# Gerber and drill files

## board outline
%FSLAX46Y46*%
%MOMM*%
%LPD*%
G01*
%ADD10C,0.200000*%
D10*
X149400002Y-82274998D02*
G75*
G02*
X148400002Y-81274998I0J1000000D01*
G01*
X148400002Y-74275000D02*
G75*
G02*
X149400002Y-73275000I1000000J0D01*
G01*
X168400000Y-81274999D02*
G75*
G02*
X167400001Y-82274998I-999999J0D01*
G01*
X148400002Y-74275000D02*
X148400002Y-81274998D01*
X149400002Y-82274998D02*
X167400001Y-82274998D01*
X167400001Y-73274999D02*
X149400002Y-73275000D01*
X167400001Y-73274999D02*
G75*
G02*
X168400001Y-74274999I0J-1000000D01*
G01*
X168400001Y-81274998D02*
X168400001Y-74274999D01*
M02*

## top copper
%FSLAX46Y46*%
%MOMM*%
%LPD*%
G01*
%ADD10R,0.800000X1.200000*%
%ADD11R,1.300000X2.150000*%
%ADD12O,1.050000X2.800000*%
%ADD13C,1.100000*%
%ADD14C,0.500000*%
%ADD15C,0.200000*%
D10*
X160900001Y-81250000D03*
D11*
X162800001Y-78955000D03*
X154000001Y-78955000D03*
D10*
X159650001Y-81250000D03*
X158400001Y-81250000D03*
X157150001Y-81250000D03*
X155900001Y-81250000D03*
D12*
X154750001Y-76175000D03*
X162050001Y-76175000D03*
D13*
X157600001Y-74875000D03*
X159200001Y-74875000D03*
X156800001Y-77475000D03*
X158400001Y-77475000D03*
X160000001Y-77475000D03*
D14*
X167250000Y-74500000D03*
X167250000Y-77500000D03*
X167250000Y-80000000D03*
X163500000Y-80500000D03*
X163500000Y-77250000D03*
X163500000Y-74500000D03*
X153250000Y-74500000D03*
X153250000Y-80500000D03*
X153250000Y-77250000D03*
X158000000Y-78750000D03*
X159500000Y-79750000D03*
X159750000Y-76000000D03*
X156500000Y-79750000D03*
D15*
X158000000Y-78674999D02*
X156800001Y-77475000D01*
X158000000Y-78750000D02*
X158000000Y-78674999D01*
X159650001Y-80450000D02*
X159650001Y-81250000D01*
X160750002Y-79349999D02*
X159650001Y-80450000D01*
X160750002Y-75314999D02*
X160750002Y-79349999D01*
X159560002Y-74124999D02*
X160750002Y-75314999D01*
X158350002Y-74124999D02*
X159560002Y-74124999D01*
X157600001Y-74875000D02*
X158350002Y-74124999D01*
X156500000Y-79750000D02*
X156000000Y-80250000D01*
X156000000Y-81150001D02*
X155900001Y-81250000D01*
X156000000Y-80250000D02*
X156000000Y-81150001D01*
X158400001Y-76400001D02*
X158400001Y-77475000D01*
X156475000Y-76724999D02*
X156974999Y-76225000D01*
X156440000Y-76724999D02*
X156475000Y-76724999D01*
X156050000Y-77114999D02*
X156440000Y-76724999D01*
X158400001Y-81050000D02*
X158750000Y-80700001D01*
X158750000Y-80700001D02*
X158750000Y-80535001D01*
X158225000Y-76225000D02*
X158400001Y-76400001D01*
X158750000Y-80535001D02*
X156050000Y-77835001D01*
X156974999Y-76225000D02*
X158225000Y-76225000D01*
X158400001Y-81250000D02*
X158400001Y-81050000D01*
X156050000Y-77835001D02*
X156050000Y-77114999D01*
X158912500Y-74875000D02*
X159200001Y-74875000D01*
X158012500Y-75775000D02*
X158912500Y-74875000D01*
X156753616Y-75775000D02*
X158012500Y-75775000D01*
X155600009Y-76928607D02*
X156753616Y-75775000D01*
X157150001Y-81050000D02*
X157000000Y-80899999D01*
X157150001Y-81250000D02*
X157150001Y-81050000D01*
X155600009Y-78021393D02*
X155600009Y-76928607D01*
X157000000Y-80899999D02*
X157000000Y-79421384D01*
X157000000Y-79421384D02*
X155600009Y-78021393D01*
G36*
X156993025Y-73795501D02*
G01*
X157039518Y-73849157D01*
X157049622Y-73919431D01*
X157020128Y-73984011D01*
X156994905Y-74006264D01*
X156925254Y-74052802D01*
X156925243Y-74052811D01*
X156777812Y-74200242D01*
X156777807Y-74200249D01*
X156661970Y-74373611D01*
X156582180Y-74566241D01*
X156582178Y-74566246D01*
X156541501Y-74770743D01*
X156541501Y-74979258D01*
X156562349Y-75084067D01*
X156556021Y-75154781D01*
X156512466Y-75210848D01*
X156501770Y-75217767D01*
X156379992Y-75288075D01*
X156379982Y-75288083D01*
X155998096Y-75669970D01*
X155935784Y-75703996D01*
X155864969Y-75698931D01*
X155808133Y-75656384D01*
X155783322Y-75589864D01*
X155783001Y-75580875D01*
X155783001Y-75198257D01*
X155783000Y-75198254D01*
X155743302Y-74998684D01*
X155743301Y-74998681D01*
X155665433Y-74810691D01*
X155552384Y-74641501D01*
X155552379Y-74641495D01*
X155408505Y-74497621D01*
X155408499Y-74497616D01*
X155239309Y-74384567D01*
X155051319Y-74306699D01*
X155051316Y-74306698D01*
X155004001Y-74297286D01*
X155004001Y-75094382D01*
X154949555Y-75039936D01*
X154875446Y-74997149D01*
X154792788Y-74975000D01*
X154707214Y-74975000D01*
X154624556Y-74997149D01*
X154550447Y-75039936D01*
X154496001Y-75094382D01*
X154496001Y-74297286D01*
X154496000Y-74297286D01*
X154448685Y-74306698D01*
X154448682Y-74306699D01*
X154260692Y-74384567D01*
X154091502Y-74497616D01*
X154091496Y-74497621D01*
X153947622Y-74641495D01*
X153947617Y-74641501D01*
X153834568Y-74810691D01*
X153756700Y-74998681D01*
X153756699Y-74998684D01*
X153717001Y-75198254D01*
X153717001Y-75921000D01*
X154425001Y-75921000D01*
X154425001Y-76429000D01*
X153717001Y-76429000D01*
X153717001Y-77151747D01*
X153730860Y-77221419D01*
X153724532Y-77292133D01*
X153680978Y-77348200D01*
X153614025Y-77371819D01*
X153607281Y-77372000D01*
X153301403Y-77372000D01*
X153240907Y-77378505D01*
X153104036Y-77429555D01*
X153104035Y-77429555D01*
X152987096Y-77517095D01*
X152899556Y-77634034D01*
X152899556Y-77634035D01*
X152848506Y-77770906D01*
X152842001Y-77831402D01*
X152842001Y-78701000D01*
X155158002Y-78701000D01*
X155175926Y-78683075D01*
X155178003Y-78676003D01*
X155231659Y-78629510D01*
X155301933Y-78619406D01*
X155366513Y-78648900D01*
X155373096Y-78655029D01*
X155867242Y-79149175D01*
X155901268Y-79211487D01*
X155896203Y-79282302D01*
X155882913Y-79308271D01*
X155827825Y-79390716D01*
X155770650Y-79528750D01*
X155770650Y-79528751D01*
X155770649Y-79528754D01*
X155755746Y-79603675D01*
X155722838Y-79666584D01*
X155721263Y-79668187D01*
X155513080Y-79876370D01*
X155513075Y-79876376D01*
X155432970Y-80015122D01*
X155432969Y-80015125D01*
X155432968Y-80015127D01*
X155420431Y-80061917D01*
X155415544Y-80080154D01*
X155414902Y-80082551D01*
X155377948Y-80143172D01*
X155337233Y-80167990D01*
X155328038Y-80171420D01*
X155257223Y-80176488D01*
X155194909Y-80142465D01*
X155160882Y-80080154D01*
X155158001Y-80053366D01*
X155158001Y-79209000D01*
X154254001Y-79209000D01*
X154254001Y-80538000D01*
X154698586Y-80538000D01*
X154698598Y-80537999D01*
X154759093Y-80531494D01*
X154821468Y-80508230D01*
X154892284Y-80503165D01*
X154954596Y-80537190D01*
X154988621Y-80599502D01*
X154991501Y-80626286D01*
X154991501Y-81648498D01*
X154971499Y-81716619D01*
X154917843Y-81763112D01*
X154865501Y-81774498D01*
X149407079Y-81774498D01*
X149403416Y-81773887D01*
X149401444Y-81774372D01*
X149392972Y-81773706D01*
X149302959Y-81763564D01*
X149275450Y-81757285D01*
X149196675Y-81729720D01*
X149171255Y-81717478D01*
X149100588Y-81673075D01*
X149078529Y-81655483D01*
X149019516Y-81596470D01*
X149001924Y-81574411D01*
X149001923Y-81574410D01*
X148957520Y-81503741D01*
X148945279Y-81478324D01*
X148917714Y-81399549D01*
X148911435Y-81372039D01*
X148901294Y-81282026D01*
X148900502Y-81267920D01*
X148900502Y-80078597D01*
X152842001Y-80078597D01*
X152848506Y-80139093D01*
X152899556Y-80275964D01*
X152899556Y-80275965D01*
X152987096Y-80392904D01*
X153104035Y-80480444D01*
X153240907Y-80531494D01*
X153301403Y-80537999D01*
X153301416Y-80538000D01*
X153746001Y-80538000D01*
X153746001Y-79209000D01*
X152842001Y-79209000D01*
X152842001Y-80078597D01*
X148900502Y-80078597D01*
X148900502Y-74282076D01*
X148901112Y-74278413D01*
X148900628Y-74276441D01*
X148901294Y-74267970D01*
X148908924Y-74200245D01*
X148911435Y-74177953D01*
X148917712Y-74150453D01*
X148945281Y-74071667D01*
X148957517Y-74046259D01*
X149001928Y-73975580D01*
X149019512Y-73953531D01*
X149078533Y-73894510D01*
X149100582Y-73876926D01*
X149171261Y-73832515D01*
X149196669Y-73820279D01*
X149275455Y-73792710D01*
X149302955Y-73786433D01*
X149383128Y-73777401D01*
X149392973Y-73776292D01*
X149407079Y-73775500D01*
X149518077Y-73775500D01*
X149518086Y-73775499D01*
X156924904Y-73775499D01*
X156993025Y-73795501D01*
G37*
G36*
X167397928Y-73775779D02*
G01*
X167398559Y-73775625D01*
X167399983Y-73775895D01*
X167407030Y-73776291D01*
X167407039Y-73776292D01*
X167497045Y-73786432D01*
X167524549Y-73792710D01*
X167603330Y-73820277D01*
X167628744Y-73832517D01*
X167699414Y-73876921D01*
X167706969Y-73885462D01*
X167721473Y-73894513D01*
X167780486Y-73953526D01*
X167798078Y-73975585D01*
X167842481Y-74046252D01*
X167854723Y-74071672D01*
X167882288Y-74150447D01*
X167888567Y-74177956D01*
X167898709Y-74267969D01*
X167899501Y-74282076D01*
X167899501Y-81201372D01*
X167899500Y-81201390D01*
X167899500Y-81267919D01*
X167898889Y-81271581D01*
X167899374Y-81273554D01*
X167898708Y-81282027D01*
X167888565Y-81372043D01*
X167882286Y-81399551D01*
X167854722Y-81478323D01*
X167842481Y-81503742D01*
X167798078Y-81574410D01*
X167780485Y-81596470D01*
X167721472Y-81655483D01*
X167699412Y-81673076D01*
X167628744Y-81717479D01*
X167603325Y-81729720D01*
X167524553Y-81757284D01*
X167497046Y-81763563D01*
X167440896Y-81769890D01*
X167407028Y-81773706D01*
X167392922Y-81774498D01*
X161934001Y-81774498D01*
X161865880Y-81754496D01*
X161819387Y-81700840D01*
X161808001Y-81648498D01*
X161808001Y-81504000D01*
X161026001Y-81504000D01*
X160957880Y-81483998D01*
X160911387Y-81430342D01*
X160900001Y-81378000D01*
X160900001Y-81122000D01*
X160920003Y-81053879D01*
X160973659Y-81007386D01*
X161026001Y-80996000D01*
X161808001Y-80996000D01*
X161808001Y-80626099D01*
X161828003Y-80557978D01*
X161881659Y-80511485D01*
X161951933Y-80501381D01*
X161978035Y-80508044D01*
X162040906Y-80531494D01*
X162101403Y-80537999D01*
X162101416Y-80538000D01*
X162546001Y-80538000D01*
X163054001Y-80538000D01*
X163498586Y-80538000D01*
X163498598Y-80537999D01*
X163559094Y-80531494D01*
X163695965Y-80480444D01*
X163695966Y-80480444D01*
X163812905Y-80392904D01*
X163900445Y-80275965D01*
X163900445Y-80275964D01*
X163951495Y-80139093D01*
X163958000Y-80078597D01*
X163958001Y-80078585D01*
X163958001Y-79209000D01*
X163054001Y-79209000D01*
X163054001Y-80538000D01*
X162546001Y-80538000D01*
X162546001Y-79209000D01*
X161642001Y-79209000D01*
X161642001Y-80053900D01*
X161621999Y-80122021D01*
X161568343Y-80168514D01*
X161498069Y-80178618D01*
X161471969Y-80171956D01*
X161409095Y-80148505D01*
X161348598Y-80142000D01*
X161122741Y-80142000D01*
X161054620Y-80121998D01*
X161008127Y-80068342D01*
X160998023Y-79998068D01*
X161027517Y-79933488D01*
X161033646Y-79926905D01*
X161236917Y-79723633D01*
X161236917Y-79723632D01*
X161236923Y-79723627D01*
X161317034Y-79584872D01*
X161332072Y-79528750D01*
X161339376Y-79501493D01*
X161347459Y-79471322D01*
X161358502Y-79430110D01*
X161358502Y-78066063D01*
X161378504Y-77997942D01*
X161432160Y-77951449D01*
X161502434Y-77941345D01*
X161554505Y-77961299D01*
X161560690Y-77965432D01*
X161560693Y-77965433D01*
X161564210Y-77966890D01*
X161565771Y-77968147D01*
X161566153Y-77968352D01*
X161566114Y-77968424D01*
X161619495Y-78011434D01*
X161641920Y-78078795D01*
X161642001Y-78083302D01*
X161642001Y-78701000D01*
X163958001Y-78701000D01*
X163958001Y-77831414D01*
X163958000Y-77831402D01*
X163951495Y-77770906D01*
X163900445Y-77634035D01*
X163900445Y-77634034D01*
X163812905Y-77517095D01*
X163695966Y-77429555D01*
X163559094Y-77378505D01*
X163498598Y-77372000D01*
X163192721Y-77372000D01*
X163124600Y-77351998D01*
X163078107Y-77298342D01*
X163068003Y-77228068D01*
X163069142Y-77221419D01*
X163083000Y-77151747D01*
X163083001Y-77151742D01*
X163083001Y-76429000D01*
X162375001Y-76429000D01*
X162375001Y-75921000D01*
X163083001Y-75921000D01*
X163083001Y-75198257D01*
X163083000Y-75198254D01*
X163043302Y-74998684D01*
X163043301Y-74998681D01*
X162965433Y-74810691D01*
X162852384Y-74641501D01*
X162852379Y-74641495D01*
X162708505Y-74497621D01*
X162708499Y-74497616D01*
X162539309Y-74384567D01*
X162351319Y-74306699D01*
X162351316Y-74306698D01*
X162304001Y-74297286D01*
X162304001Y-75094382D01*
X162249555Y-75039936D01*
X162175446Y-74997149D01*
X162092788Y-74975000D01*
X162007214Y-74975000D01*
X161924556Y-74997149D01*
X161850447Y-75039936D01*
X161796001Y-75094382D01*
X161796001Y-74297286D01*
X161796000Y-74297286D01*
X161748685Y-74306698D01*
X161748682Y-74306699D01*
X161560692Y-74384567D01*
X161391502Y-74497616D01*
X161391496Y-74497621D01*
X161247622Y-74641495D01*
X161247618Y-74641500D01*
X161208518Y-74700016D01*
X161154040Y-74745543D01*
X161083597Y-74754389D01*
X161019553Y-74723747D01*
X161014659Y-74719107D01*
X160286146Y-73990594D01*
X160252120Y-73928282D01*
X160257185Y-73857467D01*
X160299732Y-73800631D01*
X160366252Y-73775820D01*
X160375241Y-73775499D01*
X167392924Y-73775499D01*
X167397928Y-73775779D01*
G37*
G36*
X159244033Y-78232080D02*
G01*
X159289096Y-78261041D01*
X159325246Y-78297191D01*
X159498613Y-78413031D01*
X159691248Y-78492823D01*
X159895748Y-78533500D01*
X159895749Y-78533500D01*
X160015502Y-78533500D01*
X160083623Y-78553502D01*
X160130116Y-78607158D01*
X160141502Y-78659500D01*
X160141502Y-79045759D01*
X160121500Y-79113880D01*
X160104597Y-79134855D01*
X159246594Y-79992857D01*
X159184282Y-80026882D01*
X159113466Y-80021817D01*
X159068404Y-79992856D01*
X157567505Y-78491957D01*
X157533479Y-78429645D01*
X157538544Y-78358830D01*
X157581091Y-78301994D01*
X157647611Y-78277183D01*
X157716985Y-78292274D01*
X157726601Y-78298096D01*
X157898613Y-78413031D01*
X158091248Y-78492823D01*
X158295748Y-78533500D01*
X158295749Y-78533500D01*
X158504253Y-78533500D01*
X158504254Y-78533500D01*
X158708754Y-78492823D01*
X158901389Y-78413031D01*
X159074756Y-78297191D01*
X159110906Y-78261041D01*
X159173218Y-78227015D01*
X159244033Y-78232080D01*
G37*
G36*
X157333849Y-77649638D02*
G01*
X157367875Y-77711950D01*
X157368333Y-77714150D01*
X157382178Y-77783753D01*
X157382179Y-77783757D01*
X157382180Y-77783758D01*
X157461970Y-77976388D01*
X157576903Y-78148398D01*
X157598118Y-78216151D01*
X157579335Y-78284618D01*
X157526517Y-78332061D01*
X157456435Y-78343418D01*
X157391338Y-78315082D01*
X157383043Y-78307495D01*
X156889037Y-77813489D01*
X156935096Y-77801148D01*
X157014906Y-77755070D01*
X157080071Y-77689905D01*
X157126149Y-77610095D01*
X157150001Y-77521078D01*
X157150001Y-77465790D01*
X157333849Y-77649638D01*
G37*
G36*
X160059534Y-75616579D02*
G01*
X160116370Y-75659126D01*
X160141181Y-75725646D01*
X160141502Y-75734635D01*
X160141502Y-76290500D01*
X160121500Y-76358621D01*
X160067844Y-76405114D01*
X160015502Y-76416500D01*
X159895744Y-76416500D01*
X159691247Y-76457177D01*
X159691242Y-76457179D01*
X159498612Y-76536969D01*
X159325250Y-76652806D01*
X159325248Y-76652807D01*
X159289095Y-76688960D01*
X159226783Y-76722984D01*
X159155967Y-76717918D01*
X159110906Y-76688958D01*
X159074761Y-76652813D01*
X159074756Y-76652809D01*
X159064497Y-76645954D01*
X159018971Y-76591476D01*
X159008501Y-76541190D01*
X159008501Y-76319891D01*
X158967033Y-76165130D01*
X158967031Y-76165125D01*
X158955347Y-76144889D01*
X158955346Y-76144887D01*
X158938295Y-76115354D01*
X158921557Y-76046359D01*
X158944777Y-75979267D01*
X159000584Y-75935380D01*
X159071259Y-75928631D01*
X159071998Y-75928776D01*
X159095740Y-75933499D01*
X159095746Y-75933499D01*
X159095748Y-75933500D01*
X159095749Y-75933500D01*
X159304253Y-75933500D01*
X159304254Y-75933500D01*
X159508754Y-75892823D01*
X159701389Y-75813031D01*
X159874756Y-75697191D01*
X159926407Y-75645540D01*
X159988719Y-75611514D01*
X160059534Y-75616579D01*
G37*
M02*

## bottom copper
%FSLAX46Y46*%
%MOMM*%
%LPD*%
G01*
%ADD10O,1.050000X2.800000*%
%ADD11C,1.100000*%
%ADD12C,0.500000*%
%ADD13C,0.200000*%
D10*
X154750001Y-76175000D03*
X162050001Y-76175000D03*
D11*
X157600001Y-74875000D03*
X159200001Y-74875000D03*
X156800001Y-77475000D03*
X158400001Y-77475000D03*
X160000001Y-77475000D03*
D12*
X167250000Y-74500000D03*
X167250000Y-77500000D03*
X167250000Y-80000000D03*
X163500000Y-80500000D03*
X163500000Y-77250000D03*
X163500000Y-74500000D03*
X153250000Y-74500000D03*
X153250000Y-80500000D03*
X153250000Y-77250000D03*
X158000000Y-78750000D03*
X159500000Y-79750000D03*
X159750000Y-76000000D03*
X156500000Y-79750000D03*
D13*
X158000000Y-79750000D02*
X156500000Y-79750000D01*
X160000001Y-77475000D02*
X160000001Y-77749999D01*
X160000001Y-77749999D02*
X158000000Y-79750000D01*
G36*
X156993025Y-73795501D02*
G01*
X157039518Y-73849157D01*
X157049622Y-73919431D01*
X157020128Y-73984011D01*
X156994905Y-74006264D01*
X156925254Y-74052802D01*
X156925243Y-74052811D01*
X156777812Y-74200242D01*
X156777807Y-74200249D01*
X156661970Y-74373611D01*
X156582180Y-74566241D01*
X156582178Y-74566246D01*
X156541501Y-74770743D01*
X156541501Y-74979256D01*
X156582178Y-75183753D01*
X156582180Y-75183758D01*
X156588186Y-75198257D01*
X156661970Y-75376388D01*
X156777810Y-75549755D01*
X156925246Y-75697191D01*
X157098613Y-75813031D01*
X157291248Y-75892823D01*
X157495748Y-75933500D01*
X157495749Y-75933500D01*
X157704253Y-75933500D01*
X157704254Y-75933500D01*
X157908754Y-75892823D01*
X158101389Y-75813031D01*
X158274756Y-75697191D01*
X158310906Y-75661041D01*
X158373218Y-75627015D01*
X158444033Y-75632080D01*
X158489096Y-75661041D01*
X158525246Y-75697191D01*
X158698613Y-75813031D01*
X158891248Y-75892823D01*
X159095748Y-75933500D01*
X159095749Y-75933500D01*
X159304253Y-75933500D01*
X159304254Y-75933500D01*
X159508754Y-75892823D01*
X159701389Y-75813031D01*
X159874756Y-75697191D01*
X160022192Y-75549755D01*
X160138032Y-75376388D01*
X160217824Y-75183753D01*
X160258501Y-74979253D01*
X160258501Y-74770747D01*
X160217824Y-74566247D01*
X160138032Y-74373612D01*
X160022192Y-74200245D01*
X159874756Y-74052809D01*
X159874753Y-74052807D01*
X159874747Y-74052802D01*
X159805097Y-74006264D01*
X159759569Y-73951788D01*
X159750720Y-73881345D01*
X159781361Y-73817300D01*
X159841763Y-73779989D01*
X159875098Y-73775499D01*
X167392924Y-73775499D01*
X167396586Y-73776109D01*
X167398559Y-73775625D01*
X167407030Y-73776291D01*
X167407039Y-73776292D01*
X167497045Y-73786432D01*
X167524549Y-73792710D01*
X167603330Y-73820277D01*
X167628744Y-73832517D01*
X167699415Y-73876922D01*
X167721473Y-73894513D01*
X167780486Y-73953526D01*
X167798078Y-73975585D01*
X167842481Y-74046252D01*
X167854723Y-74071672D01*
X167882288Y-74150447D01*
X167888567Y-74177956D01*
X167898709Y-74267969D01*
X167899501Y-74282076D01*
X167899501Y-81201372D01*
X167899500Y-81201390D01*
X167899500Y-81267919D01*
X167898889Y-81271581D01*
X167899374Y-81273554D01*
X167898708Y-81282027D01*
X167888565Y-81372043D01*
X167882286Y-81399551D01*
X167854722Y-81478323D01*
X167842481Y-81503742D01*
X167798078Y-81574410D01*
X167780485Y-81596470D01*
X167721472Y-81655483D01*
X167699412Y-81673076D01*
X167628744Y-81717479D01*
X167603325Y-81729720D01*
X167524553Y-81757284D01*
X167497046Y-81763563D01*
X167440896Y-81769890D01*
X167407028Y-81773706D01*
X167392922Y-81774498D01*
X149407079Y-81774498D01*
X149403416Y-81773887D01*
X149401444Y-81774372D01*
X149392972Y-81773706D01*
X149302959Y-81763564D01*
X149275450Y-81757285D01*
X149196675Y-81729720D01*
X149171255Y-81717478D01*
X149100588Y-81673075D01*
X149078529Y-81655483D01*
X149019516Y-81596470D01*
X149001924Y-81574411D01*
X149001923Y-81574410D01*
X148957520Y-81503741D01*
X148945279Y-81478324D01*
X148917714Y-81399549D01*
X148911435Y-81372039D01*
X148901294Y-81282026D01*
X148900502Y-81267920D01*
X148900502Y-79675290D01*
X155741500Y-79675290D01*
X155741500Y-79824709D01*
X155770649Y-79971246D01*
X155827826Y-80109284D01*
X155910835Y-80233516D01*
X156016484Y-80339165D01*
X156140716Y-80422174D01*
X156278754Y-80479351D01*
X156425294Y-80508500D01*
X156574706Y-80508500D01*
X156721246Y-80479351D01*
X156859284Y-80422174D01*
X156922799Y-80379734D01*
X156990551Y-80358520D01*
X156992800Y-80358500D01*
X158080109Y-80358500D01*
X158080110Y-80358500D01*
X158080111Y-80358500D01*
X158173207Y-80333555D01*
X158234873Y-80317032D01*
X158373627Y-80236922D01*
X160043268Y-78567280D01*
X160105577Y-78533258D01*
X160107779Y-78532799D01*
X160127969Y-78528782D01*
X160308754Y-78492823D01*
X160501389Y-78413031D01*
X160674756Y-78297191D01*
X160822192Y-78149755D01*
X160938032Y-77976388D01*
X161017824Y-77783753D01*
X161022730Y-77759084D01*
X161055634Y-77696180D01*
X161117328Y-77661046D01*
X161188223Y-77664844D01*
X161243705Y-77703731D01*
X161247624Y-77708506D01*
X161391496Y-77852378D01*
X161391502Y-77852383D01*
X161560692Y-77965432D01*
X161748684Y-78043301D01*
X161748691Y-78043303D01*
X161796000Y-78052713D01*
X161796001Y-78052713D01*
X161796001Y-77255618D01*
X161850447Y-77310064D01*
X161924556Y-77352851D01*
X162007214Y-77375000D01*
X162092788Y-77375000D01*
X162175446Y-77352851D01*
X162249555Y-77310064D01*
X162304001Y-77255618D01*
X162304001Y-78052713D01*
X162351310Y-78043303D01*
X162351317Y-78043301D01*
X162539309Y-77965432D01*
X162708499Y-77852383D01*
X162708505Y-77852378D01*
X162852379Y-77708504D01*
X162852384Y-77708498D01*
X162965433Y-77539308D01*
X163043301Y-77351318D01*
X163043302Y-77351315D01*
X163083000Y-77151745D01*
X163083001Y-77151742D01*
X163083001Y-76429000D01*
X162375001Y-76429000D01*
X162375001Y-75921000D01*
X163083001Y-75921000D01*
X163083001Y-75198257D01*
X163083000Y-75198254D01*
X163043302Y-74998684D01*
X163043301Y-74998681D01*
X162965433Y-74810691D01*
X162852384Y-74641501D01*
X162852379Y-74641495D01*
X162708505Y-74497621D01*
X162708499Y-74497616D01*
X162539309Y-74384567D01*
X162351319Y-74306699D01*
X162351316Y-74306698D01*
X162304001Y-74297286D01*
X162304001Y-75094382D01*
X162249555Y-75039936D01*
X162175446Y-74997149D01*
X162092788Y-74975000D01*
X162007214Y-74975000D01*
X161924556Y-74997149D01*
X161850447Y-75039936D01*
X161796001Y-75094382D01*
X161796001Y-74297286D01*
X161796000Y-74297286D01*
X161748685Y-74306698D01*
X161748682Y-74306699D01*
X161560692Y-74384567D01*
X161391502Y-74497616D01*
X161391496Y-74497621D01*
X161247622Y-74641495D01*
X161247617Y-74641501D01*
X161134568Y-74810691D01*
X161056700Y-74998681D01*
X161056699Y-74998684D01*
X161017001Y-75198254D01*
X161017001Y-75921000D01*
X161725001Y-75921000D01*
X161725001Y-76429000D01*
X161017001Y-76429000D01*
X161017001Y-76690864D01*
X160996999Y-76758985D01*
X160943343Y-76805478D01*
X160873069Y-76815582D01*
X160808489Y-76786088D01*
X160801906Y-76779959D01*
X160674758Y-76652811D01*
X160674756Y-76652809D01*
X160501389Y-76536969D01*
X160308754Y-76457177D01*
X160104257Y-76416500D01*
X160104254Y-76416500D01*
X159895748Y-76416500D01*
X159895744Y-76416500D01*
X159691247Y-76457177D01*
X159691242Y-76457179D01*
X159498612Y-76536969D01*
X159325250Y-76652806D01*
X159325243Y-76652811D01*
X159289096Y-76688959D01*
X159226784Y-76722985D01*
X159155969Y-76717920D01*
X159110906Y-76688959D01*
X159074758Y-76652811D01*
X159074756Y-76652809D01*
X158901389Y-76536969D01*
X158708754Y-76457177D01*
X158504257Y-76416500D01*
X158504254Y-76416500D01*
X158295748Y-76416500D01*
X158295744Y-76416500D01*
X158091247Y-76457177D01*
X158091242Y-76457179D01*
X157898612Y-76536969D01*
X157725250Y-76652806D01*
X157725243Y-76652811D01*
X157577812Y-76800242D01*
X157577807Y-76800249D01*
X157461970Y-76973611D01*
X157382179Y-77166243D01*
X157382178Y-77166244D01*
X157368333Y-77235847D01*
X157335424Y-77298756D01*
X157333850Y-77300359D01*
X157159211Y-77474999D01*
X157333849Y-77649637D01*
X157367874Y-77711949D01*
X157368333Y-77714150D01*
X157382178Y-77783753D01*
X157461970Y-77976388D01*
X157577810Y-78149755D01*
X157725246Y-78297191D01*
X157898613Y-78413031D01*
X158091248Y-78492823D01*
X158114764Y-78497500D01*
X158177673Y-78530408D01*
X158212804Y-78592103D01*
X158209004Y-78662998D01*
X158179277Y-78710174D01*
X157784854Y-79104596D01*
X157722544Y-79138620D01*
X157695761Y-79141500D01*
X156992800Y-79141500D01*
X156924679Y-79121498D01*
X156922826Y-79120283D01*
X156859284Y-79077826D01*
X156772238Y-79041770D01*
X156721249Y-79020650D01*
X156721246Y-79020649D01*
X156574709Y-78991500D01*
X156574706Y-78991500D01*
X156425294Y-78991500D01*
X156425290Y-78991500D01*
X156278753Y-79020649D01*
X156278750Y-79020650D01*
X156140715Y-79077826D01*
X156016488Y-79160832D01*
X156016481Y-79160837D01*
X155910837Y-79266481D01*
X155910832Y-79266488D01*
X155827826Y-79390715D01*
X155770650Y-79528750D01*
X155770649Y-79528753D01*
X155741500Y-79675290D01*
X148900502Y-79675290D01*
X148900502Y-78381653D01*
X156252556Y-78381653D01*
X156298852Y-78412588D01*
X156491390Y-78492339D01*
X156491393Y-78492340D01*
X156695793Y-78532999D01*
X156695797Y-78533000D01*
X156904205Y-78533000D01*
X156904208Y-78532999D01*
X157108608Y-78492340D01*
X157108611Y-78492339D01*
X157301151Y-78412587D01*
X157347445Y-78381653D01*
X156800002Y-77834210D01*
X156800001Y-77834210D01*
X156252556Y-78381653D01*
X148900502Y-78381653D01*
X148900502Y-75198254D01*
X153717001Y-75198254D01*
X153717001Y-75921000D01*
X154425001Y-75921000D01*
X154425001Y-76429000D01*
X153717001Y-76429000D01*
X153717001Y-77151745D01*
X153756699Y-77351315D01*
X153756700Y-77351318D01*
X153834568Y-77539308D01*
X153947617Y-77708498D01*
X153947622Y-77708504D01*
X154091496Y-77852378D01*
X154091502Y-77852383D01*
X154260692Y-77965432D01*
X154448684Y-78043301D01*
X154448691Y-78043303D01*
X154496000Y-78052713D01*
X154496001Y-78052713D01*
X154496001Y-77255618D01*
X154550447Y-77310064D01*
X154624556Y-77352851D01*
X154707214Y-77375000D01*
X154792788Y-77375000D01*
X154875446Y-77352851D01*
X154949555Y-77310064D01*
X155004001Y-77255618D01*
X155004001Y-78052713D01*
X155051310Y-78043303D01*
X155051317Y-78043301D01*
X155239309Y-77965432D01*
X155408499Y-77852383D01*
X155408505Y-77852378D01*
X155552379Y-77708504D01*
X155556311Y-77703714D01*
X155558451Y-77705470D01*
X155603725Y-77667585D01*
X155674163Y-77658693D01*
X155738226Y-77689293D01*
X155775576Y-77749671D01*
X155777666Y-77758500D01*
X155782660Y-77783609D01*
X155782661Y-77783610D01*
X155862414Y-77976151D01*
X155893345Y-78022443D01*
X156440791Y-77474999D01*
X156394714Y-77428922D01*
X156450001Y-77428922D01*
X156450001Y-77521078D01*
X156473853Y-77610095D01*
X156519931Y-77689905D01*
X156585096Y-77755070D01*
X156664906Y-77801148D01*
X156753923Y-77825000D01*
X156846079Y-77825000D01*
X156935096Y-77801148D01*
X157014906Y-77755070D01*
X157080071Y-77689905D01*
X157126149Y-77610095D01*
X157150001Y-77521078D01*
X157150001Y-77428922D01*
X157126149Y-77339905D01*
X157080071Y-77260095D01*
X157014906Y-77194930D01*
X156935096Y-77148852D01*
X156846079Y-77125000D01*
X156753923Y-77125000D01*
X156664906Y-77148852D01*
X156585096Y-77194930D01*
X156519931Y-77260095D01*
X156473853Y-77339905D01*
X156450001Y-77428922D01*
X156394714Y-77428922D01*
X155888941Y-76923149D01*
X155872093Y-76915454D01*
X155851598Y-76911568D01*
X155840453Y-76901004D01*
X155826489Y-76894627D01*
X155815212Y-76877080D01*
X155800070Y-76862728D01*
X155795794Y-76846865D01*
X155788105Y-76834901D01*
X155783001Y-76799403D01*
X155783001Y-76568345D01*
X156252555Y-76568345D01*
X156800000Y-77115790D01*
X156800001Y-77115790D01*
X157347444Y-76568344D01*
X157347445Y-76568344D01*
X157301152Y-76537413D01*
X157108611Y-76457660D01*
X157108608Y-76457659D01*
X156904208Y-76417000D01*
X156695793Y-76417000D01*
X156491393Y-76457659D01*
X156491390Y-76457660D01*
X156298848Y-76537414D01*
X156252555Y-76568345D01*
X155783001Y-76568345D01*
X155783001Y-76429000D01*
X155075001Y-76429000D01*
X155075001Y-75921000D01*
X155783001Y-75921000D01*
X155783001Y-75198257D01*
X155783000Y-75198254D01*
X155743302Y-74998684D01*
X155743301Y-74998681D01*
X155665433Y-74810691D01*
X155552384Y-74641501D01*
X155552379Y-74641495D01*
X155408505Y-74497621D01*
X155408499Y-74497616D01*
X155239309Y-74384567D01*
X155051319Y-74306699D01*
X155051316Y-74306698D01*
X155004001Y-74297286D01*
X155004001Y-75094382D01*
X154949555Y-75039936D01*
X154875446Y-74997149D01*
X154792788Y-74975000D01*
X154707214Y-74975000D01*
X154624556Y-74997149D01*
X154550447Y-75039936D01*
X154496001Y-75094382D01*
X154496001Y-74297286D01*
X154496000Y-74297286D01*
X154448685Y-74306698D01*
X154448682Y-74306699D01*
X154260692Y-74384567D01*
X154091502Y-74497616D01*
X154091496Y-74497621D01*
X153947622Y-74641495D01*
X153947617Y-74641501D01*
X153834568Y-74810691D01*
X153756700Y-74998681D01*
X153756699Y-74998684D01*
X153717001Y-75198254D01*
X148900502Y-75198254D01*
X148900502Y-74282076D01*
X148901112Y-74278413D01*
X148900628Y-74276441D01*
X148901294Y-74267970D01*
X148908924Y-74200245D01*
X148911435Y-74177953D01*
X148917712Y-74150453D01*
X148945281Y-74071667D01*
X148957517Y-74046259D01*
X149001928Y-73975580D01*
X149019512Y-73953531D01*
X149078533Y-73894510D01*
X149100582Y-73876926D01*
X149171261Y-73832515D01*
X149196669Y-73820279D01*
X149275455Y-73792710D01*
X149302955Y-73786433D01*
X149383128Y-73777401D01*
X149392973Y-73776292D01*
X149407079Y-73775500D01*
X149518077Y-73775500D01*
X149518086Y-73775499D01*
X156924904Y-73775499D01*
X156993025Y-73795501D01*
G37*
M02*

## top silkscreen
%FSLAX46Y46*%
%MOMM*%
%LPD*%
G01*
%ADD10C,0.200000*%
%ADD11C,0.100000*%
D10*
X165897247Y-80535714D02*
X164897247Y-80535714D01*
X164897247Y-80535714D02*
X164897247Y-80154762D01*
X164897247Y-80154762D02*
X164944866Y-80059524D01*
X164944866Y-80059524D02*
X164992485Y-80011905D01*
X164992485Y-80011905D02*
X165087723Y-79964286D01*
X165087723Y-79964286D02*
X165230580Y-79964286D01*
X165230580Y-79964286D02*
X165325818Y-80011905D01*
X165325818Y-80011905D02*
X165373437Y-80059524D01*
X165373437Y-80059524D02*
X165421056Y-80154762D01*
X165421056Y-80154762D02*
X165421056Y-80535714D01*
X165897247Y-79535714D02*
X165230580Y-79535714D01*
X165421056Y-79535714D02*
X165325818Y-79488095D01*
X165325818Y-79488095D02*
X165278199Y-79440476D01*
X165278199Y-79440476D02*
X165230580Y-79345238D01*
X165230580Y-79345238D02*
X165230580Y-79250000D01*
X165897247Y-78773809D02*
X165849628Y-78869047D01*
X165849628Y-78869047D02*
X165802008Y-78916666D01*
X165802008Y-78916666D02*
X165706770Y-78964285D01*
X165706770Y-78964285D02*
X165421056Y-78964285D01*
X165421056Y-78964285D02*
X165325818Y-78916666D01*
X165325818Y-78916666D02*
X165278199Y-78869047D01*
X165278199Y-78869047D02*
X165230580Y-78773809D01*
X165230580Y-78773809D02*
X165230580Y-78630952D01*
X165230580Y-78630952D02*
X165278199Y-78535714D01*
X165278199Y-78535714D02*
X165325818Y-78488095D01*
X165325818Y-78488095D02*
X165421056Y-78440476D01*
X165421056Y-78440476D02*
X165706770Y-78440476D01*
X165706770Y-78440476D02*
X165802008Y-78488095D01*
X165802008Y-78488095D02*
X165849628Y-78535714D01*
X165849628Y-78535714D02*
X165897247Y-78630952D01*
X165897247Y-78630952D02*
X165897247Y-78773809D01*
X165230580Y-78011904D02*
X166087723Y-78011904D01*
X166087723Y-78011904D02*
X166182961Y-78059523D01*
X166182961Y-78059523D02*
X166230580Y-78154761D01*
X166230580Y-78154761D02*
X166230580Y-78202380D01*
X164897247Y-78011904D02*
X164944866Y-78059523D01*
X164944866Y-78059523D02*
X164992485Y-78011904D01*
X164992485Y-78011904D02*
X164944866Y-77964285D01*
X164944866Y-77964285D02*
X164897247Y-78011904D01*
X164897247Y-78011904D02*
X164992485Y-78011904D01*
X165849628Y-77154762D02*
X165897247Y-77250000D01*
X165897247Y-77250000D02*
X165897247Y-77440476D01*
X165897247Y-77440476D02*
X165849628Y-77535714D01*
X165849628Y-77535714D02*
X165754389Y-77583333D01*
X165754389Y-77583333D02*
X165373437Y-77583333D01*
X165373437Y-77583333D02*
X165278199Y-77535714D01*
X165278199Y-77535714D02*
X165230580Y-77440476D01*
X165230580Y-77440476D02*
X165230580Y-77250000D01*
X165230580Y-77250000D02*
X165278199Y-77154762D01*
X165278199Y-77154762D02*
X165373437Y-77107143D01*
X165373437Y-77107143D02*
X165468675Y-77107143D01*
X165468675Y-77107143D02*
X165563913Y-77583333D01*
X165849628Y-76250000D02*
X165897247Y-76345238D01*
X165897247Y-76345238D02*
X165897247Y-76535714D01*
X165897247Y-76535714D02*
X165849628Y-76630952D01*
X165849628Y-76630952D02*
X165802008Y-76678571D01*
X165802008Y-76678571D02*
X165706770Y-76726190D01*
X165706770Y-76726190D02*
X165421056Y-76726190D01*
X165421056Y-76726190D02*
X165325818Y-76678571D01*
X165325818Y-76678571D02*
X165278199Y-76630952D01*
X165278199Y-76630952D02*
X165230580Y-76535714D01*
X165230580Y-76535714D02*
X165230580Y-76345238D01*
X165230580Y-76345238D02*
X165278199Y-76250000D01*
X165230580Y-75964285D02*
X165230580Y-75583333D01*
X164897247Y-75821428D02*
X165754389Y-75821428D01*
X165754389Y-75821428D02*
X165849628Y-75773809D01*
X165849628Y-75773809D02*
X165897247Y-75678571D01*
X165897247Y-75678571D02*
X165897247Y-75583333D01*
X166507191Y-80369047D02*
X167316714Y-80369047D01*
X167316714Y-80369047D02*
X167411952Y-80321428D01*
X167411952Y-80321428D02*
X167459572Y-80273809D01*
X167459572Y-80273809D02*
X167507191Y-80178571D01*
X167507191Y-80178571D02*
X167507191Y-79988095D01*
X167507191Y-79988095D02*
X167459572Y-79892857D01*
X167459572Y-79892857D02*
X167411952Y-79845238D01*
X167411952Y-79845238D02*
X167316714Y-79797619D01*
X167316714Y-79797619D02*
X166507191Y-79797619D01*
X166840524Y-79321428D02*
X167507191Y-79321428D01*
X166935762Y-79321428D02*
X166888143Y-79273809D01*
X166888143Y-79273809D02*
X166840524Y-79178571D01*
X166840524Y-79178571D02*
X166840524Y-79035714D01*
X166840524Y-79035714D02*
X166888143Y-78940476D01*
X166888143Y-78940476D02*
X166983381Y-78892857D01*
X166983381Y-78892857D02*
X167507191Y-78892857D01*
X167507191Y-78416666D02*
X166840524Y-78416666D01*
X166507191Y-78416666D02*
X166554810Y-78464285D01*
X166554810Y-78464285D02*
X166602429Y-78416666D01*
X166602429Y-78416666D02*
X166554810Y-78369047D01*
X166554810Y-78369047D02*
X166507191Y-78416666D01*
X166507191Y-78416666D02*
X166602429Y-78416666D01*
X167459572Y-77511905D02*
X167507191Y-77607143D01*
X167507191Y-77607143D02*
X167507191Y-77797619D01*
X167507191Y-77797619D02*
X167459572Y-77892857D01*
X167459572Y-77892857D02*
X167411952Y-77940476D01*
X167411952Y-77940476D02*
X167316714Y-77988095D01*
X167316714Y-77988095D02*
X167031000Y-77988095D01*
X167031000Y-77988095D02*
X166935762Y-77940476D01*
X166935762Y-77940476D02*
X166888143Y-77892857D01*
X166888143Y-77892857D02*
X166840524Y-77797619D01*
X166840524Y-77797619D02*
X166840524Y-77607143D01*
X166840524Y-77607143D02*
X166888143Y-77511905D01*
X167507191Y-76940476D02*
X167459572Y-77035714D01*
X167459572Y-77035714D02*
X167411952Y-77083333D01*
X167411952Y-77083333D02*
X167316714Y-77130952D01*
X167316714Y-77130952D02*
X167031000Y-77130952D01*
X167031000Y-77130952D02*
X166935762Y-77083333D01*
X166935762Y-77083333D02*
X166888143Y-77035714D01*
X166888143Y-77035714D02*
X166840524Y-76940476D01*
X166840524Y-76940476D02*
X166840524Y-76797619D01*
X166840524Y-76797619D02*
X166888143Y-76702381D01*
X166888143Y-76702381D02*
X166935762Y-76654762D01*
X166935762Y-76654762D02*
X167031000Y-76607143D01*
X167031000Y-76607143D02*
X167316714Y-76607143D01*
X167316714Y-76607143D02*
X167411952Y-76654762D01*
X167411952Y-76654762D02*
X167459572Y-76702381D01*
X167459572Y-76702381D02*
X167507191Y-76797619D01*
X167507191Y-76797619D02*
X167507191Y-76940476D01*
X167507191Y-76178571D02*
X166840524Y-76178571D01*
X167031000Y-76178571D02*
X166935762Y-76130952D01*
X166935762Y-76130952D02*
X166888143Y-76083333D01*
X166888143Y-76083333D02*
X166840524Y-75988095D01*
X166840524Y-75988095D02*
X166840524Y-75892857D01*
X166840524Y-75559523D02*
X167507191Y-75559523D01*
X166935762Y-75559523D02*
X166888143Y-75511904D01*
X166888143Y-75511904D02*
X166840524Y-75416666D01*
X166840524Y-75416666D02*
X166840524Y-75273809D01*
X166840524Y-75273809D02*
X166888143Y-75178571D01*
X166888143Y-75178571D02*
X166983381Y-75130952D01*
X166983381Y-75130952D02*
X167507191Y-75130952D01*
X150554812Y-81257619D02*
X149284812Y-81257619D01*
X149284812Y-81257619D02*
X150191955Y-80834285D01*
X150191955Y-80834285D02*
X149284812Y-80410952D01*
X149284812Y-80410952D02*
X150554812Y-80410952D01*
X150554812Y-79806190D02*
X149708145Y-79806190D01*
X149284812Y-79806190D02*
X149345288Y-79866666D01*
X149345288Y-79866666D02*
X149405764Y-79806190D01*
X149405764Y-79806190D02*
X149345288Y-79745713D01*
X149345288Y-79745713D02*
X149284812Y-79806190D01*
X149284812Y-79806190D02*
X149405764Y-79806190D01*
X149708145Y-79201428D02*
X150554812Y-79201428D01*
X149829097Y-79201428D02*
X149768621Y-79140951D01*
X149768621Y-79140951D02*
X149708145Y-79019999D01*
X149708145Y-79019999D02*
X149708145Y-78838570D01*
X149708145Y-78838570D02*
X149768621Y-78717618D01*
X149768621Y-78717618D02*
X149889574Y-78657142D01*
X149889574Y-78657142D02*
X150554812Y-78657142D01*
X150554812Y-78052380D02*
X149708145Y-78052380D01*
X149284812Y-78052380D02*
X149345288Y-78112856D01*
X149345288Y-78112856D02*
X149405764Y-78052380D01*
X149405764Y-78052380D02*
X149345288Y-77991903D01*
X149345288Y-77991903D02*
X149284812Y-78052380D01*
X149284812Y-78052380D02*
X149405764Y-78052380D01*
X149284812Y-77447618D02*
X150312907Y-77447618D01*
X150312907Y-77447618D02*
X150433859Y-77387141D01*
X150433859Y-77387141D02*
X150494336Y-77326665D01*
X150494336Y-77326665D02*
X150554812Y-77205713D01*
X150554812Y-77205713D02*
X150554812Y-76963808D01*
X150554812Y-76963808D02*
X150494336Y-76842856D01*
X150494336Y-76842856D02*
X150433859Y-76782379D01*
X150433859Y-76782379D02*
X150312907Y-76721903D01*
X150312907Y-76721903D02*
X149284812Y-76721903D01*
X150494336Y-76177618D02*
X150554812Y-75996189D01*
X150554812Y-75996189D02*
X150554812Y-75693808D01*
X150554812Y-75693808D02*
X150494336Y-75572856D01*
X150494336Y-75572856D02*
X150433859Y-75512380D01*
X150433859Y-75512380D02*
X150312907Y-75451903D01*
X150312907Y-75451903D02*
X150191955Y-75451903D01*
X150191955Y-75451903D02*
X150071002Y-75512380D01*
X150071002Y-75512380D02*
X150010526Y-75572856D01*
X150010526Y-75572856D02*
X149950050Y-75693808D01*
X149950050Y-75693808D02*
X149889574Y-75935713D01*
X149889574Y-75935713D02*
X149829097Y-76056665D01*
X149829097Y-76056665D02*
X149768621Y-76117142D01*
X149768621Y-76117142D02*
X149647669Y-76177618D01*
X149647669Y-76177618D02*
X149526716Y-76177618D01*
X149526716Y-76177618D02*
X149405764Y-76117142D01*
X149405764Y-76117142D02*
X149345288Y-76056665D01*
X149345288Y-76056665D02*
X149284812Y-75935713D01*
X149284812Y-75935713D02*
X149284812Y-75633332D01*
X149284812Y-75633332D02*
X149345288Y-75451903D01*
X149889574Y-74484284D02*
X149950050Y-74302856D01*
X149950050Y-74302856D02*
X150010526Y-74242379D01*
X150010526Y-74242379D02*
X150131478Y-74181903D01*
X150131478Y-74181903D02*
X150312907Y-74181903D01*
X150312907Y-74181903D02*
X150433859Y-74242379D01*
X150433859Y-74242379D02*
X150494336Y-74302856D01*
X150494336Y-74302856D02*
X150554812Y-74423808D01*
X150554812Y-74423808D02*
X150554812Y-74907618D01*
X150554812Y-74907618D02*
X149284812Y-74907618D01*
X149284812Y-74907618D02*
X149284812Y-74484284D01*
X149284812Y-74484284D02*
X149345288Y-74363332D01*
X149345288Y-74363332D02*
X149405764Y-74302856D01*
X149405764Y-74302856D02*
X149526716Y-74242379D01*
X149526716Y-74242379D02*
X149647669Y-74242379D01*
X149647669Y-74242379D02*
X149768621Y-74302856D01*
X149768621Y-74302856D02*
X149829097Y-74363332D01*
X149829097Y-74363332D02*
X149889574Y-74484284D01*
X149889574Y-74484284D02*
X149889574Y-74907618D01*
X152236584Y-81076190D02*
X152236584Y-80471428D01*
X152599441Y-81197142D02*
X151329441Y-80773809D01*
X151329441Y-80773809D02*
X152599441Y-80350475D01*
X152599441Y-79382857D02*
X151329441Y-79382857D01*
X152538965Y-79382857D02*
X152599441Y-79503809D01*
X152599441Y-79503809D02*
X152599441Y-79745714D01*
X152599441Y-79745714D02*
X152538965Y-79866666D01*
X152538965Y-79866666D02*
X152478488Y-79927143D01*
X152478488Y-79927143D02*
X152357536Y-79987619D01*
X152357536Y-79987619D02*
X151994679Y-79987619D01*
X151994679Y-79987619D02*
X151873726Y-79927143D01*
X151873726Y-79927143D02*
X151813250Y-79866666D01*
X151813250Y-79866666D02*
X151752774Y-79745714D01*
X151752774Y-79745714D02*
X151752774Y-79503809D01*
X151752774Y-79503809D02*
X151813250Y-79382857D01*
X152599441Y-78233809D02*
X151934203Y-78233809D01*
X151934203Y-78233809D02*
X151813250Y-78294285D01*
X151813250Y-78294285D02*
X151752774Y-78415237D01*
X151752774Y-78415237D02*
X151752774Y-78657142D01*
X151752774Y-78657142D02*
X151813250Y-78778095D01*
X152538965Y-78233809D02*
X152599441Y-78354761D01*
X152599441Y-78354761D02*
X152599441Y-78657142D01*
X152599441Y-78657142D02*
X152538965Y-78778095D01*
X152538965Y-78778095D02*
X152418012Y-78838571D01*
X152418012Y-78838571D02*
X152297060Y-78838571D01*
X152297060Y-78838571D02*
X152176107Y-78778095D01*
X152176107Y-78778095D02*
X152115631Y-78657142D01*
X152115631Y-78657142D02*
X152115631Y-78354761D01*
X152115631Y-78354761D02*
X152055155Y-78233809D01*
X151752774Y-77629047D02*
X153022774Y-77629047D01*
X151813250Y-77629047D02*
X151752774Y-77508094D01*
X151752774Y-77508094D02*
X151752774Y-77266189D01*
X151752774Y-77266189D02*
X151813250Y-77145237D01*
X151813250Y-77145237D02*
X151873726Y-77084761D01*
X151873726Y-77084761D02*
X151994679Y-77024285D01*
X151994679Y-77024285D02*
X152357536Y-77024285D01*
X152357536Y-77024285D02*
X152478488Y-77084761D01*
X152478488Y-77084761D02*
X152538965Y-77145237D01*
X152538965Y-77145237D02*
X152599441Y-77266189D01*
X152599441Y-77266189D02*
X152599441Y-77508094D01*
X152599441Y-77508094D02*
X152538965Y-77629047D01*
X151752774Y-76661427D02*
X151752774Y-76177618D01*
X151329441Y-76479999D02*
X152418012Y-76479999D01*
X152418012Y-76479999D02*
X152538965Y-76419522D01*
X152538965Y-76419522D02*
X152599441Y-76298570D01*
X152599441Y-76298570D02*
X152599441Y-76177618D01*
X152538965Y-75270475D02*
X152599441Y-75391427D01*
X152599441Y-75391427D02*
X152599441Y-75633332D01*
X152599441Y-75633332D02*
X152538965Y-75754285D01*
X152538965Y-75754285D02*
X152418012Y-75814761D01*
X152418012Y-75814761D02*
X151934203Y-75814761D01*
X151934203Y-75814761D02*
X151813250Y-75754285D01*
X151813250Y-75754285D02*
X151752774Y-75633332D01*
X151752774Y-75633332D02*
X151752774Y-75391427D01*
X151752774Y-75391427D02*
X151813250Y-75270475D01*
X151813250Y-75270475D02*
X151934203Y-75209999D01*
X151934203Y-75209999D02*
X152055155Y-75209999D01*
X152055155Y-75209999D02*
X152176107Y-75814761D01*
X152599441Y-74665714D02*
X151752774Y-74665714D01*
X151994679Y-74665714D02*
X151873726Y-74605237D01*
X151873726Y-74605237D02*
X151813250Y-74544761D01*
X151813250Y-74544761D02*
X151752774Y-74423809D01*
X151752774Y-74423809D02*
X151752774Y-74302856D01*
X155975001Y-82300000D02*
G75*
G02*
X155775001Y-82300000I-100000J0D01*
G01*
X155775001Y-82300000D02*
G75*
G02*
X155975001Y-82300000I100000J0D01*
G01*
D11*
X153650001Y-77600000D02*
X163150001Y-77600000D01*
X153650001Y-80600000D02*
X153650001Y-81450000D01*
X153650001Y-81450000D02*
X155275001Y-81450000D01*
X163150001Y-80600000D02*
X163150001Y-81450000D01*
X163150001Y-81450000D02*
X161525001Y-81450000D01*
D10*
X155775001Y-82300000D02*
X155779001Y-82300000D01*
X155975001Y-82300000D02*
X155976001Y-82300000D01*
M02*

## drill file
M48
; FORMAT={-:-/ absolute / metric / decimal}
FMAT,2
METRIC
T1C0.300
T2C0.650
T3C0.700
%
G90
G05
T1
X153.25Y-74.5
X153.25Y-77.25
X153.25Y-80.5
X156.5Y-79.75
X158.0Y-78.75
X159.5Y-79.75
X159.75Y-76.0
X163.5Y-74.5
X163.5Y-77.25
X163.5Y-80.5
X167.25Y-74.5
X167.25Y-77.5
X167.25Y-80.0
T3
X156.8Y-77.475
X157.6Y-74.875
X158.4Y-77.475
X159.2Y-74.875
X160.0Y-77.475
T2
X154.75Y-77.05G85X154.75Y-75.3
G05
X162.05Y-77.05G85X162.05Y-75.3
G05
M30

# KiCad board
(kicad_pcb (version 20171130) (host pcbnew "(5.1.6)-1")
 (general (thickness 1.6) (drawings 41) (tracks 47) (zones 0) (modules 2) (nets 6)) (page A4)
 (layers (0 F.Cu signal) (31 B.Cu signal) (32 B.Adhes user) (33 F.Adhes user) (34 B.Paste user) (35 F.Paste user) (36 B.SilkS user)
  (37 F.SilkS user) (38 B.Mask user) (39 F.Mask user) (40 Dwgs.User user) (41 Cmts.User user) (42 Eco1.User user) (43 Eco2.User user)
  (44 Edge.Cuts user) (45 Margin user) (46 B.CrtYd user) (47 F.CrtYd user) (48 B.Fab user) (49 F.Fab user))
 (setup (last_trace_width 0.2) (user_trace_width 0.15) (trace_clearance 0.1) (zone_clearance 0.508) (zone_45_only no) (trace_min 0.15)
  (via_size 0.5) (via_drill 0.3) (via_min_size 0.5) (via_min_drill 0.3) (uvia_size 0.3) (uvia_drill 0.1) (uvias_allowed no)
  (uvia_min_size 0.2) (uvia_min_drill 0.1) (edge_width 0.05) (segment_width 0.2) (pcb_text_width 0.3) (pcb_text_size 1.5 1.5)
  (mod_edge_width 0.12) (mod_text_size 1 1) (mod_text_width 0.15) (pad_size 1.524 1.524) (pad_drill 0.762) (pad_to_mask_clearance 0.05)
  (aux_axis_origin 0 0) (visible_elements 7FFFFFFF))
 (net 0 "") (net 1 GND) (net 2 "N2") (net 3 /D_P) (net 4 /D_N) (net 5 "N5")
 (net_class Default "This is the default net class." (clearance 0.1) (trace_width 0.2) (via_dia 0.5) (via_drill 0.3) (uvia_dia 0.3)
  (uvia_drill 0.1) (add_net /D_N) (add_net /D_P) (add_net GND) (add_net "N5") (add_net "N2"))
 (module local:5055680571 (layer F.Cu) (at 158.400001 80)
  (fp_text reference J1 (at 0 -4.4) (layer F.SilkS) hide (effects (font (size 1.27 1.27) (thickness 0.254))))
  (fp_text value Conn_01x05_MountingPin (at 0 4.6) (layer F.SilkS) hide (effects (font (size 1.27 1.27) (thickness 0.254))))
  (fp_arc (start -2.525 2.3) (end -2.425 2.3) (angle 180) (layer F.SilkS) (width 0.2))
  (fp_arc (start -2.525 2.3) (end -2.625 2.3) (angle 180) (layer F.SilkS) (width 0.2))
  (fp_line (start -4.75 -2.4) (end 4.75 -2.4) (layer F.SilkS) (width 0.1))
  (fp_line (start -4.75 0.6) (end -4.75 1.45) (layer F.SilkS) (width 0.1))
  (fp_line (start -4.75 1.45) (end -3.125 1.45) (layer F.SilkS) (width 0.1))
  (fp_line (start 4.75 0.6) (end 4.75 1.45) (layer F.SilkS) (width 0.1))
  (fp_line (start 4.75 1.45) (end 3.125 1.45) (layer F.SilkS) (width 0.1))
  (fp_line (start -2.625 2.3) (end -2.621 2.3) (layer F.SilkS) (width 0.2))
  (fp_line (start -2.425 2.3) (end -2.424 2.3) (layer F.SilkS) (width 0.2))
  (pad 5 smd rect (at 2.5 1.25) (size 0.8 1.2) (layers F.Cu F.Paste F.Mask) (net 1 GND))
  (pad MP smd rect (at 4.4 -1.045) (size 1.3 2.15) (layers F.Cu F.Paste F.Mask) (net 1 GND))
  (pad MP smd rect (at -4.4 -1.045) (size 1.3 2.15) (layers F.Cu F.Paste F.Mask) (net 1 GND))
  (pad 4 smd rect (at 1.25 1.25) (size 0.8 1.2) (layers F.Cu F.Paste F.Mask) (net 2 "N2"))
  (pad 3 smd rect (at 0 1.25) (size 0.8 1.2) (layers F.Cu F.Paste F.Mask) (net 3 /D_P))
  (pad 2 smd rect (at -1.25 1.25) (size 0.8 1.2) (layers F.Cu F.Paste F.Mask) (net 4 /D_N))
  (pad 1 smd rect (at -2.5 1.25) (size 0.8 1.2) (layers F.Cu F.Paste F.Mask) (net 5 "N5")))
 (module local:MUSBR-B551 (layer B.Cu) (at 158.400001 76.175 180)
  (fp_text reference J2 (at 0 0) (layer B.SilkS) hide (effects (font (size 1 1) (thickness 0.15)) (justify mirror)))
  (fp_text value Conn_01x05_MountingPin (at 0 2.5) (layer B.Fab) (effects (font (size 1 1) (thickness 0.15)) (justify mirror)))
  (pad MP thru_hole oval (at 3.65 0 180) (size 1.05 2.8) (drill oval 0.65 2.4) (layers *.Cu *.Mask) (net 1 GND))
  (pad MP thru_hole oval (at -3.65 0 180) (size 1.05 2.8) (drill oval 0.65 2.4) (layers *.Cu *.Mask) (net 1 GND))
  (pad 4 thru_hole circle (at 0.8 1.3 180) (size 1.1 1.1) (drill 0.7) (layers *.Cu *.Mask) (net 2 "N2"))
  (pad 2 thru_hole circle (at -0.8 1.3 180) (size 1.1 1.1) (drill 0.7) (layers *.Cu *.Mask) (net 4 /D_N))
  (pad 5 thru_hole circle (at 1.6 -1.3 180) (size 1.1 1.1) (drill 0.7) (layers *.Cu *.Mask) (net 1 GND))
  (pad 3 thru_hole circle (at 0 -1.3 180) (size 1.1 1.1) (drill 0.7) (layers *.Cu *.Mask) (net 3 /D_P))
  (pad 1 thru_hole circle (at -1.6 -1.3 180) (size 1.1 1.1) (drill 0.7) (layers *.Cu *.Mask) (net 5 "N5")))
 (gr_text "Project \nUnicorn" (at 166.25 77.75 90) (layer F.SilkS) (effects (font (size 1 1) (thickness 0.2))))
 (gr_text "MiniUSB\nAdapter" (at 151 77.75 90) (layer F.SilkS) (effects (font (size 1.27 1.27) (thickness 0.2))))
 (gr_arc (start 149.400002 81.274998) (end 148.400002 81.274998) (angle -90) (layer Edge.Cuts) (width 0.2))
 (gr_arc (start 149.400002 74.275) (end 149.400002 73.275) (angle -90) (layer Edge.Cuts) (width 0.2))
 (gr_arc (start 167.400001 81.274999) (end 167.400001 82.274998) (angle -90) (layer Edge.Cuts) (width 0.2))
 (gr_line (start 148.400002 74.275) (end 148.400002 81.274998) (layer Edge.Cuts) (width 0.2))
 (gr_line (start 149.400002 82.274998) (end 167.400001 82.274998) (layer Edge.Cuts) (width 0.2))
 (gr_line (start 167.400001 73.274999) (end 149.400002 73.275) (layer Edge.Cuts) (width 0.2))
 (gr_arc (start 167.400001 74.274999) (end 168.400001 74.274999) (angle -90) (layer Edge.Cuts) (width 0.2))
 (gr_line (start 168.400001 81.274998) (end 168.400001 74.274999) (layer Edge.Cuts) (width 0.2))
 (via (at 167.25 74.5) (size 0.5) (drill 0.3) (layers F.Cu B.Cu) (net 1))
 (via (at 167.25 77.5) (size 0.5) (drill 0.3) (layers F.Cu B.Cu) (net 1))
 (via (at 167.25 80) (size 0.5) (drill 0.3) (layers F.Cu B.Cu) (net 1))
 (via (at 163.5 80.5) (size 0.5) (drill 0.3) (layers F.Cu B.Cu) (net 1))
 (via (at 163.5 77.25) (size 0.5) (drill 0.3) (layers F.Cu B.Cu) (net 1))
 (via (at 163.5 74.5) (size 0.5) (drill 0.3) (layers F.Cu B.Cu) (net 1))
 (via (at 153.25 74.5) (size 0.5) (drill 0.3) (layers F.Cu B.Cu) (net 1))
 (via (at 153.25 80.5) (size 0.5) (drill 0.3) (layers F.Cu B.Cu) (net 1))
 (via (at 153.25 77.25) (size 0.5) (drill 0.3) (layers F.Cu B.Cu) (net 1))
 (via (at 158 78.75) (size 0.5) (drill 0.3) (layers F.Cu B.Cu) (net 1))
 (via (at 159.5 79.75) (size 0.5) (drill 0.3) (layers F.Cu B.Cu) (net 1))
 (via (at 159.75 76) (size 0.5) (drill 0.3) (layers F.Cu B.Cu) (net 1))
 (segment (start 158 78.674999) (end 156.800001 77.475) (width 0.2) (layer F.Cu) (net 1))
 (segment (start 158 78.75) (end 158 78.674999) (width 0.2) (layer F.Cu) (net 1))
 (segment (start 159.650001 80.45) (end 159.650001 81.25) (width 0.2) (layer F.Cu) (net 2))
 (segment (start 160.750002 79.349999) (end 159.650001 80.45) (width 0.2) (layer F.Cu) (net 2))
 (segment (start 160.750002 75.314999) (end 160.750002 79.349999) (width 0.2) (layer F.Cu) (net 2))
 (segment (start 159.560002 74.124999) (end 160.750002 75.314999) (width 0.2) (layer F.Cu) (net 2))
 (segment (start 158.350002 74.124999) (end 159.560002 74.124999) (width 0.2) (layer F.Cu) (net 2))
 (segment (start 157.600001 74.875) (end 158.350002 74.124999) (width 0.2) (layer F.Cu) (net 2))
 (via (at 156.5 79.75) (size 0.5) (drill 0.3) (layers F.Cu B.Cu) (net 5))
 (segment (start 156.5 79.75) (end 156 80.25) (width 0.2) (layer F.Cu) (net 5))
 (segment (start 156 81.150001) (end 155.900001 81.25) (width 0.2) (layer F.Cu) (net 5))
 (segment (start 156 80.25) (end 156 81.150001) (width 0.2) (layer F.Cu) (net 5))
 (segment (start 158 79.75) (end 156.5 79.75) (width 0.2) (layer B.Cu) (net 5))
 (segment (start 160.000001 77.475) (end 160.000001 77.749999) (width 0.2) (layer B.Cu) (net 5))
 (segment (start 160.000001 77.749999) (end 158 79.75) (width 0.2) (layer B.Cu) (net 5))
 (segment (start 158.400001 76.400001) (end 158.400001 77.475) (width 0.2) (layer F.Cu) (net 3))
 (segment (start 156.475 76.724999) (end 156.974999 76.225) (width 0.2) (layer F.Cu) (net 3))
 (segment (start 156.44 76.724999) (end 156.475 76.724999) (width 0.2) (layer F.Cu) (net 3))
 (segment (start 156.05 77.114999) (end 156.44 76.724999) (width 0.2) (layer F.Cu) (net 3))
 (segment (start 158.400001 81.05) (end 158.75 80.700001) (width 0.2) (layer F.Cu) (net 3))
 (segment (start 158.75 80.700001) (end 158.75 80.535001) (width 0.2) (layer F.Cu) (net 3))
 (segment (start 158.225 76.225) (end 158.400001 76.400001) (width 0.2) (layer F.Cu) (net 3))
 (segment (start 158.75 80.535001) (end 156.05 77.835001) (width 0.2) (layer F.Cu) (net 3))
 (segment (start 156.974999 76.225) (end 158.225 76.225) (width 0.2) (layer F.Cu) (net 3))
 (segment (start 158.400001 81.25) (end 158.400001 81.05) (width 0.2) (layer F.Cu) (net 3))
 (segment (start 156.05 77.835001) (end 156.05 77.114999) (width 0.2) (layer F.Cu) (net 3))
 (segment (start 158.9125 74.875) (end 159.200001 74.875) (width 0.2) (layer F.Cu) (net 4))
 (segment (start 158.0125 75.775) (end 158.9125 74.875) (width 0.2) (layer F.Cu) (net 4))
 (segment (start 156.753616 75.775) (end 158.0125 75.775) (width 0.2) (layer F.Cu) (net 4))
 (segment (start 155.600009 76.928607) (end 156.753616 75.775) (width 0.2) (layer F.Cu) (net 4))
 (segment (start 157.150001 81.05) (end 157 80.899999) (width 0.2) (layer F.Cu) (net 4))
 (segment (start 157.150001 81.25) (end 157.150001 81.05) (width 0.2) (layer F.Cu) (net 4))
 (segment (start 155.600009 78.021393) (end 155.600009 76.928607) (width 0.2) (layer F.Cu) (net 4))
 (segment (start 157 80.899999) (end 157 79.421384) (width 0.2) (layer F.Cu) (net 4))
 (segment (start 157 79.421384) (end 155.600009 78.021393) (width 0.2) (layer F.Cu) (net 4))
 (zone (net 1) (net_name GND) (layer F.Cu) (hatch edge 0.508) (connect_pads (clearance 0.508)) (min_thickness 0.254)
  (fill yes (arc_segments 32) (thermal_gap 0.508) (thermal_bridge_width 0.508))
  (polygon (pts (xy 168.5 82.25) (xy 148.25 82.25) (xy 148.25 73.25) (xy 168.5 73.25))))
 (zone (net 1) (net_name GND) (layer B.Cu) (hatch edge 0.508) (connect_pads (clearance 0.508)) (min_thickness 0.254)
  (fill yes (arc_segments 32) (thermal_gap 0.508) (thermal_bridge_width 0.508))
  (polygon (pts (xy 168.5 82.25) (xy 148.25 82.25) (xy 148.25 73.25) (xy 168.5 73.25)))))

